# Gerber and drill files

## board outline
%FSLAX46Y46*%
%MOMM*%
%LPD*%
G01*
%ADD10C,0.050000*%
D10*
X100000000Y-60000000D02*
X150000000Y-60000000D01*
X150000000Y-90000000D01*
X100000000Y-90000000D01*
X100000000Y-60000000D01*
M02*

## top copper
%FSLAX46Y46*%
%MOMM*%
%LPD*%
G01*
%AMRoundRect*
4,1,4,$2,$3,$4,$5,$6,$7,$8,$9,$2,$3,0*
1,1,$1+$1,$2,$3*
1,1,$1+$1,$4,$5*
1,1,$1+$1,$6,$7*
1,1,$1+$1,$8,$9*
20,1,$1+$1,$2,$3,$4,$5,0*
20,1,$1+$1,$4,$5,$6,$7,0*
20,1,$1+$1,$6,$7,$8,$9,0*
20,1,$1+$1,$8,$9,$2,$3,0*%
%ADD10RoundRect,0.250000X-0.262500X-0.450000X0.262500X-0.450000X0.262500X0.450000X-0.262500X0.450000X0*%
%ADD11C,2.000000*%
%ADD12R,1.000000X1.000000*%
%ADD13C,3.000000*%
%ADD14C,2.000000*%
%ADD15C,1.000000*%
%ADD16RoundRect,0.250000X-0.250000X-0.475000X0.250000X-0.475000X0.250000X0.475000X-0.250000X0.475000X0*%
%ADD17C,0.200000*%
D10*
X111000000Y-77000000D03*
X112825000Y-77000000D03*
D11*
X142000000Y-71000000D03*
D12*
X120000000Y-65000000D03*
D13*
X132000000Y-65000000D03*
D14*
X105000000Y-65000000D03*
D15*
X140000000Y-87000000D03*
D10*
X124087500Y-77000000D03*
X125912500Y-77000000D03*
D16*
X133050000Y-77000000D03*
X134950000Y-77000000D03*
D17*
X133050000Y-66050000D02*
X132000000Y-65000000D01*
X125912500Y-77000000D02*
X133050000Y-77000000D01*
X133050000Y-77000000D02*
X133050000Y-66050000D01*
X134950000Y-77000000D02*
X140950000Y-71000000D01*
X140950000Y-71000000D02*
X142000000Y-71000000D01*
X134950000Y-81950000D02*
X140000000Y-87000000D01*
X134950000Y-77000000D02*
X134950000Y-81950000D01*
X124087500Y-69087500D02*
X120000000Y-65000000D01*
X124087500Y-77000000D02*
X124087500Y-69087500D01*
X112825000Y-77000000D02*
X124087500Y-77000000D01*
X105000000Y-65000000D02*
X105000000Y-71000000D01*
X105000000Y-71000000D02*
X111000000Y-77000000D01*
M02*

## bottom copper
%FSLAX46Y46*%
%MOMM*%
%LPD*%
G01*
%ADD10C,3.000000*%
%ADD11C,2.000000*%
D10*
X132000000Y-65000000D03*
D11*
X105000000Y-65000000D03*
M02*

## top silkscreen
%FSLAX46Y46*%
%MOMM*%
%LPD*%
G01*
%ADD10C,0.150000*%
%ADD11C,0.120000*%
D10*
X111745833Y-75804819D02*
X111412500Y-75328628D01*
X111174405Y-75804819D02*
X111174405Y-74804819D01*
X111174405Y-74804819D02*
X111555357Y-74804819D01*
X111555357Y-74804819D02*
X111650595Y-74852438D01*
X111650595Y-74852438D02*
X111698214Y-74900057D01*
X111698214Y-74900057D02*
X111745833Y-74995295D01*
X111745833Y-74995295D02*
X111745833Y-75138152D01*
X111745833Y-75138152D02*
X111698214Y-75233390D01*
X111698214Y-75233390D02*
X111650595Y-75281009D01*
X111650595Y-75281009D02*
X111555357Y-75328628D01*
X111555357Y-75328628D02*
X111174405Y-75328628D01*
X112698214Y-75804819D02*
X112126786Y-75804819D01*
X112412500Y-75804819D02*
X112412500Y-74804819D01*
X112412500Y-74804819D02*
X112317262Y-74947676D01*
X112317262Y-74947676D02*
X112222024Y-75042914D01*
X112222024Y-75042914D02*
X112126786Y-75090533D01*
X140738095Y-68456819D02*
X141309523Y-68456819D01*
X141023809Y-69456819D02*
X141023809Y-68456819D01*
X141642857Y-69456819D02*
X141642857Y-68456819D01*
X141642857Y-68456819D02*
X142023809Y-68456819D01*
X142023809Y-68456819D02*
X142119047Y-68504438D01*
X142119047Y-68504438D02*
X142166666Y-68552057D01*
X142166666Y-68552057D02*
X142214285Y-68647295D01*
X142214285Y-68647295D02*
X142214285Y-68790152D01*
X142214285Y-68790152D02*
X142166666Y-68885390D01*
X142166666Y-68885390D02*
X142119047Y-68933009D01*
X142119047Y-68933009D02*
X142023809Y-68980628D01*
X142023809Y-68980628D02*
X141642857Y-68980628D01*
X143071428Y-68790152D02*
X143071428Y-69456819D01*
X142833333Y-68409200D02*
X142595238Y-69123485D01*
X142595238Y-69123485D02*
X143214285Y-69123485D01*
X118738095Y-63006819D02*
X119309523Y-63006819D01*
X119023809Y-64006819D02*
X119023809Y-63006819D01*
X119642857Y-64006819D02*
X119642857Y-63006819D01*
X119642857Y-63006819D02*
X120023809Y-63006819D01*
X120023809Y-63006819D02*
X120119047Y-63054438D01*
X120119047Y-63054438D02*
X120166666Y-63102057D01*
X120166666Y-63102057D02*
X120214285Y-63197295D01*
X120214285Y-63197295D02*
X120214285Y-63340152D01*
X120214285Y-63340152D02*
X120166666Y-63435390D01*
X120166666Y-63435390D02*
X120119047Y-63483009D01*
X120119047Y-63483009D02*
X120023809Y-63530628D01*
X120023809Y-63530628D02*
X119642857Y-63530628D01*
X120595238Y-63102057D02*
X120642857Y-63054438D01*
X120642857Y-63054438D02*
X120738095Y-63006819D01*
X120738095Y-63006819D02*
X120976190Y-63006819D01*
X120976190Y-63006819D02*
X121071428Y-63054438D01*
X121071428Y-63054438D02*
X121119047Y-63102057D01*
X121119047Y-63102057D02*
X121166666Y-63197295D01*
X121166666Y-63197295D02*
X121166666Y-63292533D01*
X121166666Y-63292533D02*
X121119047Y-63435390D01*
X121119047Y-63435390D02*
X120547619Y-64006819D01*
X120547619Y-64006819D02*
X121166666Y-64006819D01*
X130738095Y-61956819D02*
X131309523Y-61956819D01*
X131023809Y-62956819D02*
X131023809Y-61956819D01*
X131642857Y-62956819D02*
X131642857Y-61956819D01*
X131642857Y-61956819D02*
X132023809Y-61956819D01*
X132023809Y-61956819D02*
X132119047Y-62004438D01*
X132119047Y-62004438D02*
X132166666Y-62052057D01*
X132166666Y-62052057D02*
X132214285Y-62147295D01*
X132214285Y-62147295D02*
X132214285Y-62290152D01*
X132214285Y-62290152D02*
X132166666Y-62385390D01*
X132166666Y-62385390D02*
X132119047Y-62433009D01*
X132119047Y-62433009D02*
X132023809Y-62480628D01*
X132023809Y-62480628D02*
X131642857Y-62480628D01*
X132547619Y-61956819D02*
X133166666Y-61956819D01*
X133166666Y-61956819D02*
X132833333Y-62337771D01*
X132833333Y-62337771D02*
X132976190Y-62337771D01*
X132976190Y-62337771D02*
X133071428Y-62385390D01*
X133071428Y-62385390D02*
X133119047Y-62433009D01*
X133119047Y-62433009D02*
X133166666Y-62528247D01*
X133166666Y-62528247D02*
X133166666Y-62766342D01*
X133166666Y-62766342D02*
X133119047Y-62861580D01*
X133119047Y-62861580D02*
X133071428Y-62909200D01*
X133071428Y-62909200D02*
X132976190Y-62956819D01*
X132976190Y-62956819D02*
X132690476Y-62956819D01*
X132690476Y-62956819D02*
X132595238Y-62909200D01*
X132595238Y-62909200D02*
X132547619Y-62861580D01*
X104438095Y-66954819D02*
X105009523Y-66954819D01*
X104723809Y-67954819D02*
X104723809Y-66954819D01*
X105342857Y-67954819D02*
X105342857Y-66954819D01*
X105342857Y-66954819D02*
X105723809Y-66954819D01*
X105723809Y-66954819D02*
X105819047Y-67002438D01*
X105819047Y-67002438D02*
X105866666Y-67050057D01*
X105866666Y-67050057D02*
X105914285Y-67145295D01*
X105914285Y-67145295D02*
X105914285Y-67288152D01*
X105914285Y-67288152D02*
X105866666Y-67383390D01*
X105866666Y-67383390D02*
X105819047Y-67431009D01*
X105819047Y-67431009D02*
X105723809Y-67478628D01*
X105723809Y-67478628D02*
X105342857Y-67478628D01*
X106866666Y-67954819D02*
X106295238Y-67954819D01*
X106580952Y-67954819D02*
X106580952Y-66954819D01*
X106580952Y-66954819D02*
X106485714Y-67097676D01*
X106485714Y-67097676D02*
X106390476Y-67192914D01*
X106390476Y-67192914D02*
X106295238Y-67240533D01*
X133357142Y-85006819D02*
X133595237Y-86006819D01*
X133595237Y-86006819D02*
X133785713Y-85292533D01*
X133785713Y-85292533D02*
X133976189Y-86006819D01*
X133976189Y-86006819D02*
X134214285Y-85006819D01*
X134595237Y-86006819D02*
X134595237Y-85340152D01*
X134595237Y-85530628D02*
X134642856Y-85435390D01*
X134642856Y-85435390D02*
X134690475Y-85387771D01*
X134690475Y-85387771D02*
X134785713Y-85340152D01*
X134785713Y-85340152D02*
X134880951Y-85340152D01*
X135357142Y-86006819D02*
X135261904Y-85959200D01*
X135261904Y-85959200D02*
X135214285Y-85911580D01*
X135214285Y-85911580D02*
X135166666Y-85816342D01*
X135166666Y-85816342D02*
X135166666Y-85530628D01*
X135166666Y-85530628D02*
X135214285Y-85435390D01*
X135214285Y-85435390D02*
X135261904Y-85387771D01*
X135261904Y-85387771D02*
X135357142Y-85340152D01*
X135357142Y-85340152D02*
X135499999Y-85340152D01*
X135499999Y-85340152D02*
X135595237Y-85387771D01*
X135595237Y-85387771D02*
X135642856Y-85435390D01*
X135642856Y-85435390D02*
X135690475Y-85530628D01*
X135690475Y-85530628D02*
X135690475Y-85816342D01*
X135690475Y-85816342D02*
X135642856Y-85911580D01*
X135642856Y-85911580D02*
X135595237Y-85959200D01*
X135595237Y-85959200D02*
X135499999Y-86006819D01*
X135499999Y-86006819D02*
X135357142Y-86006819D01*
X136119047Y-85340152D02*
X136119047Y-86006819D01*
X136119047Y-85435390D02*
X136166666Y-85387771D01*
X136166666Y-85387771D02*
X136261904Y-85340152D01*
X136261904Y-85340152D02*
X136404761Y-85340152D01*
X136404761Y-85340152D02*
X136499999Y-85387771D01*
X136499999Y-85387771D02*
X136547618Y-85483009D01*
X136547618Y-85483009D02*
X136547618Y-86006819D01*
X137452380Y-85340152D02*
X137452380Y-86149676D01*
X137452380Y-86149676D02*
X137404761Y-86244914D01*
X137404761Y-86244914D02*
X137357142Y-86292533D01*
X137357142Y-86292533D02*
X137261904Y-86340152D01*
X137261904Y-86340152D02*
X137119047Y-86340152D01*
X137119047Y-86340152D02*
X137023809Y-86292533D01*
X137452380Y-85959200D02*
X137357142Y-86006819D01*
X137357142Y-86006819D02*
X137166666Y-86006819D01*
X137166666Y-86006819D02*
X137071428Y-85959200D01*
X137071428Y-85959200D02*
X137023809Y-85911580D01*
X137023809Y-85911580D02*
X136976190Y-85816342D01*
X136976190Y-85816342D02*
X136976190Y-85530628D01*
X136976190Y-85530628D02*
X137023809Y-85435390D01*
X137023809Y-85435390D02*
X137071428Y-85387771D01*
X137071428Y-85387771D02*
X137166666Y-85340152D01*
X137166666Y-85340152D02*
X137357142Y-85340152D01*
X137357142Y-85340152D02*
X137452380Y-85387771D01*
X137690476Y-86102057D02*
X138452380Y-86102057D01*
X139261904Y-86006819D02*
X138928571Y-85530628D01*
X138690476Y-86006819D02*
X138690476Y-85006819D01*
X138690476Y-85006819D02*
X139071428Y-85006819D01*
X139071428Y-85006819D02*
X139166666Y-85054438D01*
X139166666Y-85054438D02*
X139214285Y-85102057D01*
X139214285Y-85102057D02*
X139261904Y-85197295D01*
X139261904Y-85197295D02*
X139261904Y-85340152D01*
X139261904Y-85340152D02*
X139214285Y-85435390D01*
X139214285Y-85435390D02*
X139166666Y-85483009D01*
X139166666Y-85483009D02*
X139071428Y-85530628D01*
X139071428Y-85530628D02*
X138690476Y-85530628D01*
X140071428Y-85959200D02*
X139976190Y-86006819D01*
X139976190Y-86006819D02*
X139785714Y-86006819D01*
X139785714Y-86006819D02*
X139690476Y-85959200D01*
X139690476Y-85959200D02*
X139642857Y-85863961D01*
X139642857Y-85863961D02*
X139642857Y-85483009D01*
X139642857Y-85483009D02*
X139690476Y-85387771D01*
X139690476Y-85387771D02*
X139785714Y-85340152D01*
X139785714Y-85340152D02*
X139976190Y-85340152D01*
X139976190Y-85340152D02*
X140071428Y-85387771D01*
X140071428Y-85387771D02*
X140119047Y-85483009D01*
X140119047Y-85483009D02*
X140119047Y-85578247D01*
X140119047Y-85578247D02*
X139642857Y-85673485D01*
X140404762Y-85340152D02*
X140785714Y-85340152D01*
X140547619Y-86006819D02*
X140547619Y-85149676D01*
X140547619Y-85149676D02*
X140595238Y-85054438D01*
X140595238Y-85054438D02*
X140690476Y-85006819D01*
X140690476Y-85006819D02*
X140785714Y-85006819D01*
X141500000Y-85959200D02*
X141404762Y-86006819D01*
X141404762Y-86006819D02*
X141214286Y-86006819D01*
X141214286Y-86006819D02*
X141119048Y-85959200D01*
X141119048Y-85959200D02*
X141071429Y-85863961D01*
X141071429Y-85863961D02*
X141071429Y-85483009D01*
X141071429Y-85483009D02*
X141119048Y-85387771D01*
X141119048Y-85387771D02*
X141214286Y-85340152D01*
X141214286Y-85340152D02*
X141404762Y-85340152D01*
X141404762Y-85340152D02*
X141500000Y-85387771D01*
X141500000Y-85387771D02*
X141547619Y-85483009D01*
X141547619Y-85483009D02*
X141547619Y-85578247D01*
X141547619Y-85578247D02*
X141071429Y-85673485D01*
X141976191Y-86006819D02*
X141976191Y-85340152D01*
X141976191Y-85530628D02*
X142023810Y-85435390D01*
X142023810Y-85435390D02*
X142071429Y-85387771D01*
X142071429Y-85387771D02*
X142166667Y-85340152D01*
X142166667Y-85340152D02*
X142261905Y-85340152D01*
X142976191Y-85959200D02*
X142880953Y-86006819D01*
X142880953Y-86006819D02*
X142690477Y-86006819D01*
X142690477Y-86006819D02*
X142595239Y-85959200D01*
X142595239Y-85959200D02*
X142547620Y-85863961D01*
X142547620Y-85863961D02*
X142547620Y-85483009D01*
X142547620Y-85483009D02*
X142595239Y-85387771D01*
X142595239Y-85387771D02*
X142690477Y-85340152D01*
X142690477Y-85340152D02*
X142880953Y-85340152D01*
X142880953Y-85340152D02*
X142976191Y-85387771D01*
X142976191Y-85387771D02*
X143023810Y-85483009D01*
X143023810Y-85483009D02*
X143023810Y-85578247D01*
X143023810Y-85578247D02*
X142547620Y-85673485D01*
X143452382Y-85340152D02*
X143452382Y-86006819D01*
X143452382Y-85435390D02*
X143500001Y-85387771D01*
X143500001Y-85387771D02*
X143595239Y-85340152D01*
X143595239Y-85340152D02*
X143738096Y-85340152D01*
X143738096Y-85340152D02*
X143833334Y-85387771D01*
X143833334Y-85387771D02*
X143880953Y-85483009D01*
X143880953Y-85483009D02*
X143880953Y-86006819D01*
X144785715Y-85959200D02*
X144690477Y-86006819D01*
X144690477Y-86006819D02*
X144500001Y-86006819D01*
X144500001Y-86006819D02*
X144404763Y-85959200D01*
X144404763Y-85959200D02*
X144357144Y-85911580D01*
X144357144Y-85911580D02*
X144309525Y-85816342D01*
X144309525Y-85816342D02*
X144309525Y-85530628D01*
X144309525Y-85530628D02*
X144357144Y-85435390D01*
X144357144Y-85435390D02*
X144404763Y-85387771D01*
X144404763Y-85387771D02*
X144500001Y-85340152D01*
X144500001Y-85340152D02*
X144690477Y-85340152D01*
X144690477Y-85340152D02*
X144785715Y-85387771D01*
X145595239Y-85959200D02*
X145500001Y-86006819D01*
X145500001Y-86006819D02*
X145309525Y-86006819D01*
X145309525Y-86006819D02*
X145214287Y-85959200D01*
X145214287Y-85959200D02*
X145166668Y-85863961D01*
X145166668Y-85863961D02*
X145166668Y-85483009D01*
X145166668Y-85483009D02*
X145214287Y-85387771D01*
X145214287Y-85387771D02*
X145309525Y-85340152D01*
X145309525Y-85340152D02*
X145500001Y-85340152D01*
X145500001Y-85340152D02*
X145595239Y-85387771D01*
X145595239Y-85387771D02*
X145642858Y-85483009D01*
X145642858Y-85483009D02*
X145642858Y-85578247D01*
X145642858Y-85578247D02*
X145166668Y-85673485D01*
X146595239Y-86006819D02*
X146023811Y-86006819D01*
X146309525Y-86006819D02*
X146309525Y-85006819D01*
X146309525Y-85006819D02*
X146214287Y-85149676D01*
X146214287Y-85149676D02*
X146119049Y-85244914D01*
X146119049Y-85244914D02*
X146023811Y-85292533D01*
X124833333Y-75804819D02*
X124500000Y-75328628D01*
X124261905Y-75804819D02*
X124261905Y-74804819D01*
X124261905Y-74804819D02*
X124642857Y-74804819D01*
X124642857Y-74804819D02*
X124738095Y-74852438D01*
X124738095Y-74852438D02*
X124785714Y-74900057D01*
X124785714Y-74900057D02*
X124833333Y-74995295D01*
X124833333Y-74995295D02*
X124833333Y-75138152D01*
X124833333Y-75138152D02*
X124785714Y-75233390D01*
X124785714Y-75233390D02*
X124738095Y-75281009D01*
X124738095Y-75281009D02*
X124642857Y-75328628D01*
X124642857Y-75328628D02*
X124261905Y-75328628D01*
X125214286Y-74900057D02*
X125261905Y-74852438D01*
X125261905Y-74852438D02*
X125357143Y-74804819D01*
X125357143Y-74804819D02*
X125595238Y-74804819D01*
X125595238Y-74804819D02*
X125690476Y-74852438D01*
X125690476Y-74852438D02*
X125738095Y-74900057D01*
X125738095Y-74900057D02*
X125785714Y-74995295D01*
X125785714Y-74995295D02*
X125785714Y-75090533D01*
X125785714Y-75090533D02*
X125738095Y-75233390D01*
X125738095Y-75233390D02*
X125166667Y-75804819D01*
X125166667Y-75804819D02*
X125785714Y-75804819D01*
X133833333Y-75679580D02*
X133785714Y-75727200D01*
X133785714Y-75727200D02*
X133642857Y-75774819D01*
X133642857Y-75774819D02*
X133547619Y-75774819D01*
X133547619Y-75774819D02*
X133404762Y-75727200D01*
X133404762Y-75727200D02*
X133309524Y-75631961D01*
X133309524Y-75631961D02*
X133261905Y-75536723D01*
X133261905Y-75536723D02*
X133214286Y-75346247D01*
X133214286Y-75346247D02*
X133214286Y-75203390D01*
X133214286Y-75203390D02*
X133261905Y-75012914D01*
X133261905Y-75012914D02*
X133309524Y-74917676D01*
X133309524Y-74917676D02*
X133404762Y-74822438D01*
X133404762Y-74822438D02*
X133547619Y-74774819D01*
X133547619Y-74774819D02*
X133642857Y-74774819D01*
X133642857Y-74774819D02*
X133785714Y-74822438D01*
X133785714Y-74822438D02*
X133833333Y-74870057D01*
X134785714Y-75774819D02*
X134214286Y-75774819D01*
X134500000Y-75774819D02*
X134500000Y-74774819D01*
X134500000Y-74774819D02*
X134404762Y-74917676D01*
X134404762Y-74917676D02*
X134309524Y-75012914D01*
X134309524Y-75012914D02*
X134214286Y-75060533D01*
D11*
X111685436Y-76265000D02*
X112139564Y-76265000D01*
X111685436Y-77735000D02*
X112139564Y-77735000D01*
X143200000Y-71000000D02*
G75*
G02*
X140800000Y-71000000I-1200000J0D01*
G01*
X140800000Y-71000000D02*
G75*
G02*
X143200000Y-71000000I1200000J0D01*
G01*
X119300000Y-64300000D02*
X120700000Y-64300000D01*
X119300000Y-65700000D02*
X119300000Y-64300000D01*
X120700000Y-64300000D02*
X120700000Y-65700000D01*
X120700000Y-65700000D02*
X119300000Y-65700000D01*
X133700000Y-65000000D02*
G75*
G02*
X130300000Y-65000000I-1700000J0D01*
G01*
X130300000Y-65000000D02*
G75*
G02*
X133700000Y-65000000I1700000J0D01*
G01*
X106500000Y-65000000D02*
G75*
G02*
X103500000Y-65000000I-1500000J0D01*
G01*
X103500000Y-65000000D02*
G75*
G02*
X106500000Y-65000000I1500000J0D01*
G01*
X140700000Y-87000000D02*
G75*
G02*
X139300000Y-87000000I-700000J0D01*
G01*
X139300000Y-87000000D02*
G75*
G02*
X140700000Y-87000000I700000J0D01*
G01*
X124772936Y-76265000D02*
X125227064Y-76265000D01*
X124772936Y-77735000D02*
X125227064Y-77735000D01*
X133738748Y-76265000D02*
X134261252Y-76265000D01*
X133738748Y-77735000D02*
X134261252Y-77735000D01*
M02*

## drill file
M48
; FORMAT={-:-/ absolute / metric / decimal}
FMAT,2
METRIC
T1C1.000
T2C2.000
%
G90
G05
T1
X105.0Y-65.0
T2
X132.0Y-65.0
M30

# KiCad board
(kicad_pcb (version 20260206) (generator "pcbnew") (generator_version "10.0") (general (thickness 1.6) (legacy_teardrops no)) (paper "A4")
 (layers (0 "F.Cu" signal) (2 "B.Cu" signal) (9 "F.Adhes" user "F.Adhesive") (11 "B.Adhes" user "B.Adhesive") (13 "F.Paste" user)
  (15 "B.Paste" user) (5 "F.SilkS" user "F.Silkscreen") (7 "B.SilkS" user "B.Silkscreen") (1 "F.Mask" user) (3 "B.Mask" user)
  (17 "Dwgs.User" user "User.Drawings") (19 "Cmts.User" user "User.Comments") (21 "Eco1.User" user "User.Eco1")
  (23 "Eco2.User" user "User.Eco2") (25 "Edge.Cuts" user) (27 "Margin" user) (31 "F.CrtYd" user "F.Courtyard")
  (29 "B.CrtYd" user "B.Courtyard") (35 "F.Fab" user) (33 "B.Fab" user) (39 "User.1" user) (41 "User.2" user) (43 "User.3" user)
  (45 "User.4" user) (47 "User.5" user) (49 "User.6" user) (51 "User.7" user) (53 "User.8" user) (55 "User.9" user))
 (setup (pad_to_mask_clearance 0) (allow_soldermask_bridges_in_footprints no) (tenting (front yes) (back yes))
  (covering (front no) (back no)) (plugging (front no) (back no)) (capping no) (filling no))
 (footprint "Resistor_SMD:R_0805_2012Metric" (layer "F.Cu") (at 111.9125 77)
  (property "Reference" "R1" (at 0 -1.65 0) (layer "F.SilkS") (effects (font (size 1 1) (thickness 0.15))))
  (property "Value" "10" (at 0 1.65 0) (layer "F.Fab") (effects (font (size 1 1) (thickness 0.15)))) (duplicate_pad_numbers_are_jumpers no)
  (fp_line (start -0.227064 -0.735) (end 0.227064 -0.735) (stroke (width 0.12) (type solid)) (layer "F.SilkS"))
  (fp_line (start -0.227064 0.735) (end 0.227064 0.735) (stroke (width 0.12) (type solid)) (layer "F.SilkS"))
  (pad "1" smd roundrect (at -0.9125 0) (size 1.025 1.4) (layers "F.Cu" "F.Mask" "F.Paste") (roundrect_rratio 0.243902)
   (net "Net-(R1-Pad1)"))
  (pad "2" smd roundrect (at 0.9125 0) (size 1.025 1.4) (layers "F.Cu" "F.Mask" "F.Paste") (roundrect_rratio 0.243902) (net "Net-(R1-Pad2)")))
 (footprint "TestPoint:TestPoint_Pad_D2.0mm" (layer "F.Cu") (at 142 71)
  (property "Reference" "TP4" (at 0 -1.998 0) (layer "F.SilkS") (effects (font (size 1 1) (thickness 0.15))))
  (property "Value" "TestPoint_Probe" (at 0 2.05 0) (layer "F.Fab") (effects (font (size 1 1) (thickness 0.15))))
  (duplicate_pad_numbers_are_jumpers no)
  (fp_circle (center 0 0) (end 0 1.2) (stroke (width 0.12) (type solid)) (fill no) (layer "F.SilkS"))
  (pad "1" smd circle (at 0 0) (size 2 2) (layers "F.Cu" "F.Mask") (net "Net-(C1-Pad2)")))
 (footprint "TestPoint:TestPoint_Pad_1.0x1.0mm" (layer "F.Cu") (at 120 65)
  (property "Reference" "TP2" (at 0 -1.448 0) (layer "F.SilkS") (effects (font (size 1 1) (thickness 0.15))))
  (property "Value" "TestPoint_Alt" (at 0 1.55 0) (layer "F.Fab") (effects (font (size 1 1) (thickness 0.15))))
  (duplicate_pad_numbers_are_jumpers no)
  (fp_line (start -0.7 -0.7) (end 0.7 -0.7) (stroke (width 0.12) (type solid)) (layer "F.SilkS"))
  (fp_line (start -0.7 0.7) (end -0.7 -0.7) (stroke (width 0.12) (type solid)) (layer "F.SilkS"))
  (fp_line (start 0.7 -0.7) (end 0.7 0.7) (stroke (width 0.12) (type solid)) (layer "F.SilkS"))
  (fp_line (start 0.7 0.7) (end -0.7 0.7) (stroke (width 0.12) (type solid)) (layer "F.SilkS"))
  (pad "1" smd rect (at 0 0) (size 1 1) (layers "F.Cu" "F.Mask") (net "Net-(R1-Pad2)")))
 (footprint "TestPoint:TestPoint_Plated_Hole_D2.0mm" (layer "F.Cu") (at 132 65)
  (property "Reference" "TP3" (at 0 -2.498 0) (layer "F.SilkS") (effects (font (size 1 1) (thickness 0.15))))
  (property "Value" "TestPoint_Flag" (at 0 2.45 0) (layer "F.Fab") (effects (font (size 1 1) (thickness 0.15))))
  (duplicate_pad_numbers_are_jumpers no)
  (fp_circle (center 0 0) (end 0 -1.7) (stroke (width 0.12) (type solid)) (fill no) (layer "F.SilkS"))
  (pad "1" thru_hole circle (at 0 0) (size 3 3) (drill 2) (layers "*.Cu" "*.Mask") (remove_unused_layers no) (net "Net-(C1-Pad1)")))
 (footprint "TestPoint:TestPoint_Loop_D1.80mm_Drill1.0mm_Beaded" (layer "F.Cu") (at 105 65)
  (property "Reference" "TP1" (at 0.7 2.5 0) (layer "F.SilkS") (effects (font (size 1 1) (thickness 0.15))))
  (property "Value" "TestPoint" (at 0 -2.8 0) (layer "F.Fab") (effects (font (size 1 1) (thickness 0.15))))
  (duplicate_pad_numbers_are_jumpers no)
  (fp_circle (center 0 0) (end 1.5 0) (stroke (width 0.12) (type solid)) (fill no) (layer "F.SilkS"))
  (pad "1" thru_hole circle (at 0 0) (size 2 2) (drill 1) (layers "*.Cu" "*.Mask") (remove_unused_layers no) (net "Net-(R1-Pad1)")))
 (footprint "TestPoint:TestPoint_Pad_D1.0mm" (layer "F.Cu") (at 140 87)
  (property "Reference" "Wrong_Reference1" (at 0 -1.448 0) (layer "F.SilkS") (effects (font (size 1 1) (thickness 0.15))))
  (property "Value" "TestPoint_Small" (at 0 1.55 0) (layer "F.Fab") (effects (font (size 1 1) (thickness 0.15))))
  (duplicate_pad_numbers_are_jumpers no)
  (fp_circle (center 0 0) (end 0 0.7) (stroke (width 0.12) (type solid)) (fill no) (layer "F.SilkS"))
  (pad "1" smd circle (at 0 0) (size 1 1) (layers "F.Cu" "F.Mask") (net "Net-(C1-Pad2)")))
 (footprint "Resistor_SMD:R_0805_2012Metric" (layer "F.Cu") (at 125 77)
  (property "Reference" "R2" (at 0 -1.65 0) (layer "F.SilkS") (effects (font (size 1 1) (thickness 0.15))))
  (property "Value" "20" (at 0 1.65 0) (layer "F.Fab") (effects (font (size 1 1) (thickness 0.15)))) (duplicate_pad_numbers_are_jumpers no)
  (fp_line (start -0.227064 -0.735) (end 0.227064 -0.735) (stroke (width 0.12) (type solid)) (layer "F.SilkS"))
  (fp_line (start -0.227064 0.735) (end 0.227064 0.735) (stroke (width 0.12) (type solid)) (layer "F.SilkS"))
  (pad "1" smd roundrect (at -0.9125 0) (size 1.025 1.4) (layers "F.Cu" "F.Mask" "F.Paste") (roundrect_rratio 0.243902)
   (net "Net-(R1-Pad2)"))
  (pad "2" smd roundrect (at 0.9125 0) (size 1.025 1.4) (layers "F.Cu" "F.Mask" "F.Paste") (roundrect_rratio 0.243902) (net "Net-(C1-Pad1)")))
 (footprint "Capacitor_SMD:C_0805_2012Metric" (layer "F.Cu") (at 134 77)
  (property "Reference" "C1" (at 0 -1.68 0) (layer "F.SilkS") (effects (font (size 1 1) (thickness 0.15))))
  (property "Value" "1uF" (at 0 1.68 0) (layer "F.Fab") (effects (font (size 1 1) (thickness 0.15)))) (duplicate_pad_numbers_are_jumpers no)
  (fp_line (start -0.261252 -0.735) (end 0.261252 -0.735) (stroke (width 0.12) (type solid)) (layer "F.SilkS"))
  (fp_line (start -0.261252 0.735) (end 0.261252 0.735) (stroke (width 0.12) (type solid)) (layer "F.SilkS"))
  (pad "1" smd roundrect (at -0.95 0) (size 1 1.45) (layers "F.Cu" "F.Mask" "F.Paste") (roundrect_rratio 0.25) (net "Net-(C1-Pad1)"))
  (pad "2" smd roundrect (at 0.95 0) (size 1 1.45) (layers "F.Cu" "F.Mask" "F.Paste") (roundrect_rratio 0.25) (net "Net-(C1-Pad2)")))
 (gr_rect (start 100 60) (end 150 90) (stroke (width 0.05) (type default)) (fill no) (layer "Edge.Cuts"))
 (segment (start 133.05 66.05) (end 132 65) (width 0.2) (layer "F.Cu") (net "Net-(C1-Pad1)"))
 (segment (start 125.9125 77) (end 133.05 77) (width 0.2) (layer "F.Cu") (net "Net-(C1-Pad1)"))
 (segment (start 133.05 77) (end 133.05 66.05) (width 0.2) (layer "F.Cu") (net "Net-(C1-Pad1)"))
 (segment (start 134.95 77) (end 140.95 71) (width 0.2) (layer "F.Cu") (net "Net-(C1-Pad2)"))
 (segment (start 140.95 71) (end 142 71) (width 0.2) (layer "F.Cu") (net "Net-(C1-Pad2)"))
 (segment (start 134.95 81.95) (end 140 87) (width 0.2) (layer "F.Cu") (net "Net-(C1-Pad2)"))
 (segment (start 134.95 77) (end 134.95 81.95) (width 0.2) (layer "F.Cu") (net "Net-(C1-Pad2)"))
 (segment (start 124.0875 69.0875) (end 120 65) (width 0.2) (layer "F.Cu") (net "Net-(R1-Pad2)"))
 (segment (start 124.0875 77) (end 124.0875 69.0875) (width 0.2) (layer "F.Cu") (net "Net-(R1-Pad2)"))
 (segment (start 112.825 77) (end 124.0875 77) (width 0.2) (layer "F.Cu") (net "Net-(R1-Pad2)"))
 (segment (start 105 65) (end 105 71) (width 0.2) (layer "F.Cu") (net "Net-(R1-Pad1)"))
 (segment (start 105 71) (end 111 77) (width 0.2) (layer "F.Cu") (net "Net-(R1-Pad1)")))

